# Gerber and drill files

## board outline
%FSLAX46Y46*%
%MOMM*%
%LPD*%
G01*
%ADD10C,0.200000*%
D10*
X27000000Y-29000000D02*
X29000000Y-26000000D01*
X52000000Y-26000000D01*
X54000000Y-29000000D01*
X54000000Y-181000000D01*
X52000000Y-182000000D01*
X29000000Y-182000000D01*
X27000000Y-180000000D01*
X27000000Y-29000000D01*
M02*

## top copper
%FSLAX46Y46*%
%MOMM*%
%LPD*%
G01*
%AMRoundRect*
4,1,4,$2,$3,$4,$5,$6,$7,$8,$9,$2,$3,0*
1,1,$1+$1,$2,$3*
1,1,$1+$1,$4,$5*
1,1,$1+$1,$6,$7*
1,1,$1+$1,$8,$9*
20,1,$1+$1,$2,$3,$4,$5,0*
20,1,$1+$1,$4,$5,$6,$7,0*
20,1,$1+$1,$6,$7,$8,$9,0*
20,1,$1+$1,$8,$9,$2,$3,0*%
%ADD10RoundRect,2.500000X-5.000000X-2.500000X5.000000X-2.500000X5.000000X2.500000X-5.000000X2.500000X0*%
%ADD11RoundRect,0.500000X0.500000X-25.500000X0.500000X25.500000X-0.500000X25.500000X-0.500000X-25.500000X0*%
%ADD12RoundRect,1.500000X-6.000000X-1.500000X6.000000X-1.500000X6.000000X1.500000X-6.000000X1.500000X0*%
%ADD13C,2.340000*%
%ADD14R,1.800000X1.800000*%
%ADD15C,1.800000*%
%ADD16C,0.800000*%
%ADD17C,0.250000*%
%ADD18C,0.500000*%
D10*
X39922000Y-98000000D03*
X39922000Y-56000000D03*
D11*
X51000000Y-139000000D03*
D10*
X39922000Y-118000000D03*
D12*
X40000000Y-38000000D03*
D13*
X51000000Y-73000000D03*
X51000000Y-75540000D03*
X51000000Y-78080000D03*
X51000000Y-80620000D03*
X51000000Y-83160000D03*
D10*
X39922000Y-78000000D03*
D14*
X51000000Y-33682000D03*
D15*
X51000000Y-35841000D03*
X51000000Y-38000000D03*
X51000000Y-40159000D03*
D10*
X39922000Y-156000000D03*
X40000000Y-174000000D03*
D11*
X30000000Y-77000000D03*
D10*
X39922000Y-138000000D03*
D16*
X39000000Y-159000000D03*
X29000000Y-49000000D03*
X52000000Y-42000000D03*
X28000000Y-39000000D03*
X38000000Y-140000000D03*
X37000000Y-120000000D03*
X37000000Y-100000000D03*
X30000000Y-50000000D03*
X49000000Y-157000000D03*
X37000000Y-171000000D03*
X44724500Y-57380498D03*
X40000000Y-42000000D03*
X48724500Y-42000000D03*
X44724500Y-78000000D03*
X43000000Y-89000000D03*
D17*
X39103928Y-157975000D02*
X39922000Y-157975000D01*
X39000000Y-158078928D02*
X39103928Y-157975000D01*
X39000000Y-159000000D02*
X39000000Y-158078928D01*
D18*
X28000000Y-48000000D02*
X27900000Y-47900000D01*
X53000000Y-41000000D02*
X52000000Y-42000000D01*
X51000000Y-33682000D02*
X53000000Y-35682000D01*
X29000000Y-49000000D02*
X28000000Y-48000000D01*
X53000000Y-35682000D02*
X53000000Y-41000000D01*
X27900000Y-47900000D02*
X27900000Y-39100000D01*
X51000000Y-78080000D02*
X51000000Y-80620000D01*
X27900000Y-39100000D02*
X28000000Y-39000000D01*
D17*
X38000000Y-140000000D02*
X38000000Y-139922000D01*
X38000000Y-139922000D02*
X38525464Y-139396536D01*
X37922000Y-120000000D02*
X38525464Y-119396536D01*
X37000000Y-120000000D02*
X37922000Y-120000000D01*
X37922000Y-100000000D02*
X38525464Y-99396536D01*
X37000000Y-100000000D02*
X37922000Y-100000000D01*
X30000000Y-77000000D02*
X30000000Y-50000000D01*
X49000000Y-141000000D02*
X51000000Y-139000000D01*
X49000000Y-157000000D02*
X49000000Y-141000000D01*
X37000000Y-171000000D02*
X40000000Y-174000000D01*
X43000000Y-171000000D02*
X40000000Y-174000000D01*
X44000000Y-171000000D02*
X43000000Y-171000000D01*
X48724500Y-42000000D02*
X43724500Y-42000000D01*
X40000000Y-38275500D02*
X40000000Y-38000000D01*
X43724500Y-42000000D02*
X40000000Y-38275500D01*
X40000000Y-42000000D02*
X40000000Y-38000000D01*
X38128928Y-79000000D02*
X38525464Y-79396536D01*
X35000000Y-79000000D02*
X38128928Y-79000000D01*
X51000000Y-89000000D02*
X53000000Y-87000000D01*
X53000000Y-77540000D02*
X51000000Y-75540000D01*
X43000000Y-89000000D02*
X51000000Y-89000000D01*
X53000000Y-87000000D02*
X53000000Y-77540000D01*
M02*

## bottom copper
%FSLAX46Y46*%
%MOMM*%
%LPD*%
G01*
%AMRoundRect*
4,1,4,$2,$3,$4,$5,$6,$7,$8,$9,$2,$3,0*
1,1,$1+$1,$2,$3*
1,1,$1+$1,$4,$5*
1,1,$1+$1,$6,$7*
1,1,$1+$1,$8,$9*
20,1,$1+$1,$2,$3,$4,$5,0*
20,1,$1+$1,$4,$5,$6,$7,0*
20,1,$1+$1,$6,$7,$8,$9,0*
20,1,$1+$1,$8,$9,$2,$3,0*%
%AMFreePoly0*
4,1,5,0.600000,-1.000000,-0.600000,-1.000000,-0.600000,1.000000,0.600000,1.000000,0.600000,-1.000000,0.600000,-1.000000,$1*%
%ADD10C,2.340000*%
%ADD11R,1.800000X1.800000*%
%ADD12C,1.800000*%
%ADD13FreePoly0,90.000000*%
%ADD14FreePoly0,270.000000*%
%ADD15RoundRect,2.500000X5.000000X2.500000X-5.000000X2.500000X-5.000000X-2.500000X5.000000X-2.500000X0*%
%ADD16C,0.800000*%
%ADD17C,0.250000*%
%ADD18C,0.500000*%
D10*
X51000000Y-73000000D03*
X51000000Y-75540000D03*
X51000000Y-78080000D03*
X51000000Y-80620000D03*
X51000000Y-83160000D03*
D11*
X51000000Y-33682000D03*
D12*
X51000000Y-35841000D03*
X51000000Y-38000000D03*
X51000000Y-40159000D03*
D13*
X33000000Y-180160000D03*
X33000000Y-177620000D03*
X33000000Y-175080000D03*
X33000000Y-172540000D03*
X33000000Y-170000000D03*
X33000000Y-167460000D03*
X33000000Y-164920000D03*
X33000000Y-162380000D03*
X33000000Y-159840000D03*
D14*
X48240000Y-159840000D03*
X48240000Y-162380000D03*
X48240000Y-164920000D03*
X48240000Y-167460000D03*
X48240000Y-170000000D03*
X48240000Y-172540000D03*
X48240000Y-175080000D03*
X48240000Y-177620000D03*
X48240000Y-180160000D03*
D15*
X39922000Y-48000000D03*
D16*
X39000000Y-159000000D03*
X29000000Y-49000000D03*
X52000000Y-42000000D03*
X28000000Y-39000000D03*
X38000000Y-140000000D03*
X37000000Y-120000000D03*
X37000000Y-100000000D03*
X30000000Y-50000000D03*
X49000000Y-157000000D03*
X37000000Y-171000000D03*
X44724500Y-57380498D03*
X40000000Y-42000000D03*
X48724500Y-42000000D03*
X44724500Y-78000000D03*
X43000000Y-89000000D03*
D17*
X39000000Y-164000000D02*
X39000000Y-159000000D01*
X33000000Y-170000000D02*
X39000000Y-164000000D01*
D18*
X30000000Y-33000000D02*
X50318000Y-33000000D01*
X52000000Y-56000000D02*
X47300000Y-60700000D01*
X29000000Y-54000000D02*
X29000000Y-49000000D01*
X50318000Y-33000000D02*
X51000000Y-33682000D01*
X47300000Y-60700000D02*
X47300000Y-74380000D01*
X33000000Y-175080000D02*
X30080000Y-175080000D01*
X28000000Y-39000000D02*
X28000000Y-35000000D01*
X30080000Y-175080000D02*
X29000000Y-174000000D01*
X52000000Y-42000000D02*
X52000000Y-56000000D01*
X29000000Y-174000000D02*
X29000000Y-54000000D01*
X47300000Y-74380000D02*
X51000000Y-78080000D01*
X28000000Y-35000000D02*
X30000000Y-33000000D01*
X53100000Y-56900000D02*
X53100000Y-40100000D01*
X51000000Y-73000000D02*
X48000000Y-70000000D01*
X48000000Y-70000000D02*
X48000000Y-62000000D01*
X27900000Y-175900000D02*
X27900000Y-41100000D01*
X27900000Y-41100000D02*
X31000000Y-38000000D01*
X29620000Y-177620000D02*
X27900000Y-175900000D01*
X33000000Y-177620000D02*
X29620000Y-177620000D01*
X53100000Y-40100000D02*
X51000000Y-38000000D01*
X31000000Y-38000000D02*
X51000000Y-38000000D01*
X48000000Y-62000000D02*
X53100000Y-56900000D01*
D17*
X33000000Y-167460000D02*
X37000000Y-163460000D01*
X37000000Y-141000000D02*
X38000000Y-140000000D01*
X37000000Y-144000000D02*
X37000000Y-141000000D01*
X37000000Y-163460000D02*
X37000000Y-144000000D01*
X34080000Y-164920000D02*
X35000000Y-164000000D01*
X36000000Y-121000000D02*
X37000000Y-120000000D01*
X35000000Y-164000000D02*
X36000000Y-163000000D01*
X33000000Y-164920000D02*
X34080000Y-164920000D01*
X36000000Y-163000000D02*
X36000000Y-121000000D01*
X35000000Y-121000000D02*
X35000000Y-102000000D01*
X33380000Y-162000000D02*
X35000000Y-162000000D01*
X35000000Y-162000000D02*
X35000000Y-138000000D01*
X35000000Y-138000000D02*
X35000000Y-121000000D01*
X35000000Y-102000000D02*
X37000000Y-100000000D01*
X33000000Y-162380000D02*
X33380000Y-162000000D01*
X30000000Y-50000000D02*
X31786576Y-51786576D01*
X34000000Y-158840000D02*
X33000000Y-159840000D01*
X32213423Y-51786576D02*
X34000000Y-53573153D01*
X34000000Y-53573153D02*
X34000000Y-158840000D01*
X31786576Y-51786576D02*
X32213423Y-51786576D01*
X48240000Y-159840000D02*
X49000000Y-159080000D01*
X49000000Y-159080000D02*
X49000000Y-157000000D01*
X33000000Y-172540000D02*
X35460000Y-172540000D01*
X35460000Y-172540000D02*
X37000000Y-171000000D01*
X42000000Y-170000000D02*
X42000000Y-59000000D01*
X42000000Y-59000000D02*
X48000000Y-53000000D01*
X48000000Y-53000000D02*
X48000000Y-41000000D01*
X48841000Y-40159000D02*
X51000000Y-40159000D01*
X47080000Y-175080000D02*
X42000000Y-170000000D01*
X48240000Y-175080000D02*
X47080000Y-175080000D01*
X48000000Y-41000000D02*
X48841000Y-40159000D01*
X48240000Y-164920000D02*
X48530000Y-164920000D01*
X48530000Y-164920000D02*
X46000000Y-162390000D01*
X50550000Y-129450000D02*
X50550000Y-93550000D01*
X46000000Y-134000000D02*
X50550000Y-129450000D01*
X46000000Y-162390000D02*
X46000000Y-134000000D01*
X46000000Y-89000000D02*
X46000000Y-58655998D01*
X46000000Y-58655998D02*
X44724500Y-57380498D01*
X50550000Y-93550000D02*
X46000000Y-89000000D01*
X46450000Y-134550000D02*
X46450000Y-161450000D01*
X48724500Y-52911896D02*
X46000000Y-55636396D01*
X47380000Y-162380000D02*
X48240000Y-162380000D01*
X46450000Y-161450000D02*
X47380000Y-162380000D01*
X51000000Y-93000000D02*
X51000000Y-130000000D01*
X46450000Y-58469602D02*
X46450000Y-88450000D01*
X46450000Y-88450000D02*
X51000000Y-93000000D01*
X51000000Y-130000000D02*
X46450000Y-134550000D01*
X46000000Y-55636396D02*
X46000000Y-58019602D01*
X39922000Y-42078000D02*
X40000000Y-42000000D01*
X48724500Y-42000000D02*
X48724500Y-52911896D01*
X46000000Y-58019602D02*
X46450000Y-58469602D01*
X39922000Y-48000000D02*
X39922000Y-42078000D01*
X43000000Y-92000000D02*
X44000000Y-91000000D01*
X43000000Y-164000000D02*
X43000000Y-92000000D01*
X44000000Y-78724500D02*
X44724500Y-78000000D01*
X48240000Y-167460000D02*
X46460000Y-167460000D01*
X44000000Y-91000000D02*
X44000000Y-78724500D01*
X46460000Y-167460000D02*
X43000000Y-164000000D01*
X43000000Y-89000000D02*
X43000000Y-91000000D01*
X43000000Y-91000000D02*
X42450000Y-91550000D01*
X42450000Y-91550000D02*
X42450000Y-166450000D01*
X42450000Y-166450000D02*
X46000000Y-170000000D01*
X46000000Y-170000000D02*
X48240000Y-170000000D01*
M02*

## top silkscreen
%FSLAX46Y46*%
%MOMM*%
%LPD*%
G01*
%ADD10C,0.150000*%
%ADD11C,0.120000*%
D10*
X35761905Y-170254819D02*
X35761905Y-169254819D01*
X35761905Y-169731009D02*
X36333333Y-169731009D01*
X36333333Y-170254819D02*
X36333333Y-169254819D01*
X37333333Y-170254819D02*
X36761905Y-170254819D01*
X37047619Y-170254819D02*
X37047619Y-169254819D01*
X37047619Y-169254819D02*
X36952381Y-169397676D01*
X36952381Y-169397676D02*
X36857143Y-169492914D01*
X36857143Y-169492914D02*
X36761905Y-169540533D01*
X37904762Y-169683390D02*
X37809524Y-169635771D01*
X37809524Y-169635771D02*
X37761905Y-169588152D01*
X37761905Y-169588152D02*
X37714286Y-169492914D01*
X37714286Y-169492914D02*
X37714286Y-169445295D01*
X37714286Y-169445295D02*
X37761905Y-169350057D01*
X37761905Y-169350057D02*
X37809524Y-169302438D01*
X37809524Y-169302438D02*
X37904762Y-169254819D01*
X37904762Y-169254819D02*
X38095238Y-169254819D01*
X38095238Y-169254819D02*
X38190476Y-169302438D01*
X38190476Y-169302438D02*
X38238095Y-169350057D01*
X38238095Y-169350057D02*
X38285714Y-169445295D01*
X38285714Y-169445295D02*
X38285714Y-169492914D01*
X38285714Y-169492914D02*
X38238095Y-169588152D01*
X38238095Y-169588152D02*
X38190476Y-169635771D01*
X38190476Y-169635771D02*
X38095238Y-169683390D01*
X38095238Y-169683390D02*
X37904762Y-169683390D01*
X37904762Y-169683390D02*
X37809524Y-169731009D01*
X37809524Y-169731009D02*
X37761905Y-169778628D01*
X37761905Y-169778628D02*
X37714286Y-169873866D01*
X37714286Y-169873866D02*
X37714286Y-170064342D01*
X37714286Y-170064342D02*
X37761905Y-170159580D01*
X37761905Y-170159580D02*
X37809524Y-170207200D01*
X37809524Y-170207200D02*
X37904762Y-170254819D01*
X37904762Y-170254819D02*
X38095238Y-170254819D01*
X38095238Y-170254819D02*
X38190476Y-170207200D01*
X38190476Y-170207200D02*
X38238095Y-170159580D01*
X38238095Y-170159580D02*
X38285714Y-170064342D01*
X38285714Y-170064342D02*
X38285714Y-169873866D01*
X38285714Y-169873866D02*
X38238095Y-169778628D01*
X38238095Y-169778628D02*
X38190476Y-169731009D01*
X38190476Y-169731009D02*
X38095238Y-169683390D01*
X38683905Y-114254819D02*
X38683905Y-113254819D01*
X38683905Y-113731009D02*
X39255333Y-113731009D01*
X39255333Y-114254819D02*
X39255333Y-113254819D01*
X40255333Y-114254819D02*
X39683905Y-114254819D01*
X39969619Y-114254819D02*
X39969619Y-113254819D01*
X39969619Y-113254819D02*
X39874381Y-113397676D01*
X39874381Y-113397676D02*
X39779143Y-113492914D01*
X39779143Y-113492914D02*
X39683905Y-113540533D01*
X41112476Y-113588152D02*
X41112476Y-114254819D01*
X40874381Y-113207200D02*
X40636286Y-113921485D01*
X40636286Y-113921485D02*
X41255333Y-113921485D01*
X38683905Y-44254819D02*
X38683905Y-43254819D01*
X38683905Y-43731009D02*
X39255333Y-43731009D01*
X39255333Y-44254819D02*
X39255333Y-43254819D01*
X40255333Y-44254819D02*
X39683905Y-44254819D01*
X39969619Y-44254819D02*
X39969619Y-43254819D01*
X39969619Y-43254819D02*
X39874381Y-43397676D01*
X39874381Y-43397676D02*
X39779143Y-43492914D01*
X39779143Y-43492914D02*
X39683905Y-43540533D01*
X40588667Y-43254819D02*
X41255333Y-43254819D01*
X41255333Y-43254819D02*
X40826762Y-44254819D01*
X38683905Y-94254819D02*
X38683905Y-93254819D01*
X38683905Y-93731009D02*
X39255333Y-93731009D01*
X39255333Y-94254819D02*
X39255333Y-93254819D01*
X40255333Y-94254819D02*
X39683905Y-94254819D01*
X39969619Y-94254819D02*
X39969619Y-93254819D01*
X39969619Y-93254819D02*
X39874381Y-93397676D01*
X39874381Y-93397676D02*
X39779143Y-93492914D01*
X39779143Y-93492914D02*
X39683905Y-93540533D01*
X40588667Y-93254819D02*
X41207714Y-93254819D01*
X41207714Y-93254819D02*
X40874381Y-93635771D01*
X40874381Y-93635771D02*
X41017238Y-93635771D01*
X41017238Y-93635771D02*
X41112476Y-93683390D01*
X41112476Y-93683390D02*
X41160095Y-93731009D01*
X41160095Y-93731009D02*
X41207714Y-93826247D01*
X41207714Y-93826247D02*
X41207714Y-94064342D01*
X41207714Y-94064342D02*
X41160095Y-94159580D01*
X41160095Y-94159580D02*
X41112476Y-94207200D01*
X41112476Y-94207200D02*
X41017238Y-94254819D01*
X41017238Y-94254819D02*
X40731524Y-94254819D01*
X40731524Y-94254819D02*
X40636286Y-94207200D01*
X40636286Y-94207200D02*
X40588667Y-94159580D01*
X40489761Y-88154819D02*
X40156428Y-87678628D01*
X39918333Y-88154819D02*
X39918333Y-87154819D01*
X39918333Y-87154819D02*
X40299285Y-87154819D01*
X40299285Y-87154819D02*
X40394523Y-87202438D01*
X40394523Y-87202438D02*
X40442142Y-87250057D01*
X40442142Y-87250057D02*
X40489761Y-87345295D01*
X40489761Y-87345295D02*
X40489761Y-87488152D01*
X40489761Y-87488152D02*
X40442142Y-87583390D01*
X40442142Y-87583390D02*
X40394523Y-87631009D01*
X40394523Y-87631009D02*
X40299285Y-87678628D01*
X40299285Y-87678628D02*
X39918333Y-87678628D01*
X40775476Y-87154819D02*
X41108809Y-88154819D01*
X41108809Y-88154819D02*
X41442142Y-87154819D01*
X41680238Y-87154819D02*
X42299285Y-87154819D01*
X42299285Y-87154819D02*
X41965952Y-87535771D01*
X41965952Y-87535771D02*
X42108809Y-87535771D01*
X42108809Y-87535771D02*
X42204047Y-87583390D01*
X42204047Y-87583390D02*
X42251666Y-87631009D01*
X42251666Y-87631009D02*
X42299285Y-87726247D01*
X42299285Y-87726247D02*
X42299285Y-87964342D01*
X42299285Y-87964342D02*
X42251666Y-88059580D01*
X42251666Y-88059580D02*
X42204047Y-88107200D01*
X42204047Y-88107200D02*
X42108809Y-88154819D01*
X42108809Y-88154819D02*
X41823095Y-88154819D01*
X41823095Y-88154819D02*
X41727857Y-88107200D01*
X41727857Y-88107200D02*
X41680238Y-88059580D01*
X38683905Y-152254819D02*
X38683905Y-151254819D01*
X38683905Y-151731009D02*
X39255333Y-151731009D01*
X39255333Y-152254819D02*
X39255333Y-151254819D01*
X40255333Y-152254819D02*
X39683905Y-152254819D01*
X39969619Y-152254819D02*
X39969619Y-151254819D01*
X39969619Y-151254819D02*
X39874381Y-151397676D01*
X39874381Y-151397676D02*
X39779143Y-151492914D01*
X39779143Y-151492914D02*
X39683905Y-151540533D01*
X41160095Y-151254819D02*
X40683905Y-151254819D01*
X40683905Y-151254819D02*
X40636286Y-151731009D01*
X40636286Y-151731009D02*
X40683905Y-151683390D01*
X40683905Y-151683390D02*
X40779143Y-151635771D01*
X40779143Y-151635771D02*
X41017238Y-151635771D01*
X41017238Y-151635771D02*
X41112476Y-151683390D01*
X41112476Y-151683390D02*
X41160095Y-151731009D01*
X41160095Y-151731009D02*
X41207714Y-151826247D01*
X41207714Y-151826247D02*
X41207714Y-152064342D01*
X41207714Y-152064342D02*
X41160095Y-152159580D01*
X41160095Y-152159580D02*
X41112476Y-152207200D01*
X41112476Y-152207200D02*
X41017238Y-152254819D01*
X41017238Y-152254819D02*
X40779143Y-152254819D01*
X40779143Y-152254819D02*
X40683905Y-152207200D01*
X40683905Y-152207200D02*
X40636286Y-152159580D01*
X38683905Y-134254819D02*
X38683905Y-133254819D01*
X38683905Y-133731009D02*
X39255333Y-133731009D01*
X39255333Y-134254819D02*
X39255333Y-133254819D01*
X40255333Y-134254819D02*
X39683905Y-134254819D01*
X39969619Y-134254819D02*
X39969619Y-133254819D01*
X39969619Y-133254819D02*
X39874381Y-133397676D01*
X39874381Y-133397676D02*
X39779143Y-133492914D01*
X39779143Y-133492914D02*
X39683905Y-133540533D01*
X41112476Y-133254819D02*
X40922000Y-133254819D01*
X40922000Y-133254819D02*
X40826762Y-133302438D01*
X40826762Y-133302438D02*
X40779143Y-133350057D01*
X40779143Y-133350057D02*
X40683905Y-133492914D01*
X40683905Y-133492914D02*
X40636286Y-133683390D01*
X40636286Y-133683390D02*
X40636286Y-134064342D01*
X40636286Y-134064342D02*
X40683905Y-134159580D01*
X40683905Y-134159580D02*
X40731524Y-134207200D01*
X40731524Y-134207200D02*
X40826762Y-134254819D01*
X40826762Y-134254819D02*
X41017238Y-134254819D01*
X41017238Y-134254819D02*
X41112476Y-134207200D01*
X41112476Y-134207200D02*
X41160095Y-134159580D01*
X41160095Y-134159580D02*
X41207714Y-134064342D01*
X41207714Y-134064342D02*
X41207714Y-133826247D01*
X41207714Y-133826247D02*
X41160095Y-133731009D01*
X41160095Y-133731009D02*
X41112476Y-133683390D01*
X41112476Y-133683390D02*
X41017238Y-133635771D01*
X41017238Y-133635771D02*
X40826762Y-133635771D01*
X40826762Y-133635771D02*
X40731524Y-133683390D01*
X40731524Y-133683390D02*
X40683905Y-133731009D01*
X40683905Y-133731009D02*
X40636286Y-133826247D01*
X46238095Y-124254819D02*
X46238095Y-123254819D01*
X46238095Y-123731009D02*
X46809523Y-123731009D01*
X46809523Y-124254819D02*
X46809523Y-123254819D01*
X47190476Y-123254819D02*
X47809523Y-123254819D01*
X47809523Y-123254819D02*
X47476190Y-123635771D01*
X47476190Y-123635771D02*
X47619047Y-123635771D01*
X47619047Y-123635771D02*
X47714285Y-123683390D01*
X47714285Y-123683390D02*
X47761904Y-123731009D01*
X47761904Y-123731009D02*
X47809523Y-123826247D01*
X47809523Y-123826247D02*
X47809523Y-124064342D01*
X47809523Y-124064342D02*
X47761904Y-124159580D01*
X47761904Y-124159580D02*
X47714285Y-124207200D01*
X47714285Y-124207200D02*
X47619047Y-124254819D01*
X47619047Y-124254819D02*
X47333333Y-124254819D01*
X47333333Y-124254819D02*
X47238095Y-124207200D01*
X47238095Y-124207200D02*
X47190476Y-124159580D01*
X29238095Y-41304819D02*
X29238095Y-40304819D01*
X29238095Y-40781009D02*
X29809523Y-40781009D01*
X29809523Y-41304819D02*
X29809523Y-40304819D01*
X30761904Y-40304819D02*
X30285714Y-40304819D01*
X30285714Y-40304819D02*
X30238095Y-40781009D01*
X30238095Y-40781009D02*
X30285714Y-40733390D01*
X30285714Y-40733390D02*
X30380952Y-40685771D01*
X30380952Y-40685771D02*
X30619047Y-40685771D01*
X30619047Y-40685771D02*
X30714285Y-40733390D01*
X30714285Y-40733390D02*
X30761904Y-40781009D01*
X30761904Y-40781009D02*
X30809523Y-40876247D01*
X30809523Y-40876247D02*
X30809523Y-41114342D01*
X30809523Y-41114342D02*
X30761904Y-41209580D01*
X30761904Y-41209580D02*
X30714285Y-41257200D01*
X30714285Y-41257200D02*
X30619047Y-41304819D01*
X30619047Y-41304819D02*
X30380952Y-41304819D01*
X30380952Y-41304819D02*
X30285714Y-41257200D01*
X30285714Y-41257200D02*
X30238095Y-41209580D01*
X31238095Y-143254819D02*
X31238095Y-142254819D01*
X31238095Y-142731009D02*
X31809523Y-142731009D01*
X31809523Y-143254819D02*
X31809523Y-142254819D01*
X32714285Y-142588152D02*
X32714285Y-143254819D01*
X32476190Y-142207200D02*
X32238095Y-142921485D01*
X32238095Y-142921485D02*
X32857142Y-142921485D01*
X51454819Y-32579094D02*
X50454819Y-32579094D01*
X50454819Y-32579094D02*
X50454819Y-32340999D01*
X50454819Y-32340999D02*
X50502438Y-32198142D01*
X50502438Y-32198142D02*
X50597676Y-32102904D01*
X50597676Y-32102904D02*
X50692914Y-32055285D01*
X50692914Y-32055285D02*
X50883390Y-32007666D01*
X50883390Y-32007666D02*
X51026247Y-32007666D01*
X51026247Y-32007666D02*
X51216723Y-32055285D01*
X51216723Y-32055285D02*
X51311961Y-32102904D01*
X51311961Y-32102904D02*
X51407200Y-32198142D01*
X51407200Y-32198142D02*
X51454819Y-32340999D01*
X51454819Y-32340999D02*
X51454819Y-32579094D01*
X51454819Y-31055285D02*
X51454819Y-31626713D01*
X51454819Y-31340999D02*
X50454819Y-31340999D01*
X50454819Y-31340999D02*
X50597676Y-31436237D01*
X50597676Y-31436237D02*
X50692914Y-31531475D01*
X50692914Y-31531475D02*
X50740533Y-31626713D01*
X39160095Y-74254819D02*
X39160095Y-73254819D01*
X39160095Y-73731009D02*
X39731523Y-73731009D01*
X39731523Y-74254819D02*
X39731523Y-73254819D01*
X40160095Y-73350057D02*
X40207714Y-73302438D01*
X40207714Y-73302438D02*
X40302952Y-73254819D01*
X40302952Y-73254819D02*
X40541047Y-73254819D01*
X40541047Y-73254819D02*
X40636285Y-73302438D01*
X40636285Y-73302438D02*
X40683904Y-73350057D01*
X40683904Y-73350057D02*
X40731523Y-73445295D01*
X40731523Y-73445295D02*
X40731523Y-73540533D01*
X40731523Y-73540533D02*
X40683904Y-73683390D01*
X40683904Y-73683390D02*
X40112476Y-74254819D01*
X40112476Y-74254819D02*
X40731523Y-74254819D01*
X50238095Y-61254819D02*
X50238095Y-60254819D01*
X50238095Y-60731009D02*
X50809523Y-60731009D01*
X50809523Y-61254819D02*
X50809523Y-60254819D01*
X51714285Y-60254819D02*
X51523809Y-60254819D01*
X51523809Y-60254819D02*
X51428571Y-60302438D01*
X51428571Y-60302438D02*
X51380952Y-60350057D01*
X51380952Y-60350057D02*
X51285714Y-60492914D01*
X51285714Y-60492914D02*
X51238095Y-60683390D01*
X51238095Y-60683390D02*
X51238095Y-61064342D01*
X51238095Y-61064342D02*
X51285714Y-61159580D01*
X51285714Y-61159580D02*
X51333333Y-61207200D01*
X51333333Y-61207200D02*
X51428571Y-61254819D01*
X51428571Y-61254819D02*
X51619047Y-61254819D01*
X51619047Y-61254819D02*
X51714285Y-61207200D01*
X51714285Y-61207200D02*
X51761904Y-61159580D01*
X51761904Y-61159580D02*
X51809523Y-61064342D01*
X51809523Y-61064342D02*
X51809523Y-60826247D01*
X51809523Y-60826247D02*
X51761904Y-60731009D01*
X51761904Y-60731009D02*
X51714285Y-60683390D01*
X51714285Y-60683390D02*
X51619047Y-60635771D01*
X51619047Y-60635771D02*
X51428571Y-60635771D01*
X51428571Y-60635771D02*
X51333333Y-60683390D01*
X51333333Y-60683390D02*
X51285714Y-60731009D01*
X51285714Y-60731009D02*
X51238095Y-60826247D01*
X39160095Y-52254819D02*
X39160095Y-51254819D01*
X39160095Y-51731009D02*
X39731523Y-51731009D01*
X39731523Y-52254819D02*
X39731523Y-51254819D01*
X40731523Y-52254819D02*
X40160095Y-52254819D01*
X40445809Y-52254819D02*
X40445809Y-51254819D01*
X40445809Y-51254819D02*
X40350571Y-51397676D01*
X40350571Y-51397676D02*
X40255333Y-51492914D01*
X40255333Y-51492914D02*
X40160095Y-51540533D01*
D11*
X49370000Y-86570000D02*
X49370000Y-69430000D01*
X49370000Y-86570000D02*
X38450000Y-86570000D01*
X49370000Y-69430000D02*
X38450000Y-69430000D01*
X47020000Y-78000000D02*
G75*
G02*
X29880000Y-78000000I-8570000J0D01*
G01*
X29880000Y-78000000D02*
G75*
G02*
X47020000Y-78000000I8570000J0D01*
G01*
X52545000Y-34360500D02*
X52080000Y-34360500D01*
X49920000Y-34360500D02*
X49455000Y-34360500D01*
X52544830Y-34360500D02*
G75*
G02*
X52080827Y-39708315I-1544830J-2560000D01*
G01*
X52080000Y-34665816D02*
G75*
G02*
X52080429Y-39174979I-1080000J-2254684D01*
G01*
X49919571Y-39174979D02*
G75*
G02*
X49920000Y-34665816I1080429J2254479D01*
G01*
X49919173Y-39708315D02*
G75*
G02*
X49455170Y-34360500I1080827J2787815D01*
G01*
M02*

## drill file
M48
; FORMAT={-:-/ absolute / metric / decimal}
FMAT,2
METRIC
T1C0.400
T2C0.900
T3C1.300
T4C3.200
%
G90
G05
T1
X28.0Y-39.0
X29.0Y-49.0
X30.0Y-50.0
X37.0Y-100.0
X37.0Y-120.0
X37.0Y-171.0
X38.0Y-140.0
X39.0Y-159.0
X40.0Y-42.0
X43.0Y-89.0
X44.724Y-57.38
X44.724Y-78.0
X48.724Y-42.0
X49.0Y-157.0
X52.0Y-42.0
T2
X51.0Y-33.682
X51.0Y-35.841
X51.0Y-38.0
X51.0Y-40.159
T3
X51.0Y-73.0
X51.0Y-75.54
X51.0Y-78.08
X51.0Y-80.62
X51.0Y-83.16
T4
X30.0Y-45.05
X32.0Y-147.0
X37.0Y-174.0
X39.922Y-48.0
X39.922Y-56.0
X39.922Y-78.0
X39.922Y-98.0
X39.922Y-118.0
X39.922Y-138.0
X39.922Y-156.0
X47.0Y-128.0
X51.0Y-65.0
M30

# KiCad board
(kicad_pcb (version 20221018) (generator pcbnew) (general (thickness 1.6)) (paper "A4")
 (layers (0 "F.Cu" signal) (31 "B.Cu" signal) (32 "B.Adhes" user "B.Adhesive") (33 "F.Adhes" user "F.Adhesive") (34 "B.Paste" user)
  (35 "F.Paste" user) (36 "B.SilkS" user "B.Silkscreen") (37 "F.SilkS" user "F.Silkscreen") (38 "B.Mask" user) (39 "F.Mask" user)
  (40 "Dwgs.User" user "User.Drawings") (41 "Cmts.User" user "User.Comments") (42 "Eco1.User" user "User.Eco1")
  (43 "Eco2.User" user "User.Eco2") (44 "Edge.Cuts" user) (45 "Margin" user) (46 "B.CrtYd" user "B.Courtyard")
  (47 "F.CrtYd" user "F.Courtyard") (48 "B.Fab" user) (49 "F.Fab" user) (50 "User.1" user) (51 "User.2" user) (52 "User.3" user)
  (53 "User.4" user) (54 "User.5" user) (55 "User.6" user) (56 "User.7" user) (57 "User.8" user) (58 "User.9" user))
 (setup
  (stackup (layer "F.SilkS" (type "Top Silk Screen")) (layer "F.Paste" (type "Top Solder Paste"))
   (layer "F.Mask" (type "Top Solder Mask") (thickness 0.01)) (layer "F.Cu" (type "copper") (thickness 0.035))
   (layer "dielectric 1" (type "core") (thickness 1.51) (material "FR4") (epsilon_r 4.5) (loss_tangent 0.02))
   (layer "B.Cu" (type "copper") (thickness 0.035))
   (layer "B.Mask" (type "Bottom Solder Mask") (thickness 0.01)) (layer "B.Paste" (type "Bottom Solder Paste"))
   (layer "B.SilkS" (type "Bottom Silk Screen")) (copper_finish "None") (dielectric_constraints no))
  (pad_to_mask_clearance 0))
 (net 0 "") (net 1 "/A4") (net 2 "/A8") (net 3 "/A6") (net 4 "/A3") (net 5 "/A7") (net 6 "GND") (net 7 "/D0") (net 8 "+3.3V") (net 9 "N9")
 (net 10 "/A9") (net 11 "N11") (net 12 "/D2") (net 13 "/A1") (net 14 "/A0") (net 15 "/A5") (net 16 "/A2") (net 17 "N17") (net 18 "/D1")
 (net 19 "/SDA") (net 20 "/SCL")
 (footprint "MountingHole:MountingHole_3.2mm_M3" (layer "F.Cu") (at 37 174)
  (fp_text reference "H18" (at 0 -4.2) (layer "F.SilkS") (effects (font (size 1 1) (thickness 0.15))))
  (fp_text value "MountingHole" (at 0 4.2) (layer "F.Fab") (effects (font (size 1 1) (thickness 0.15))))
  (pad "" np_thru_hole circle (at 0 0) (size 3.2 3.2) (drill 3.2) (layers "*.Cu" "*.Mask")))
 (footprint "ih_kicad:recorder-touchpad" (layer "F.Cu") (at 39.922 98)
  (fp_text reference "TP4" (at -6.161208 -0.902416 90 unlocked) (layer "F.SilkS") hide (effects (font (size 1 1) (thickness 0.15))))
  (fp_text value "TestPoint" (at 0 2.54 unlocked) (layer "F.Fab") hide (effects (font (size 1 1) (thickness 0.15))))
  (pad "1" smd roundrect (at 0 0) (size 15 10) (layers "F.Cu" "F.Mask") (roundrect_rratio 0.25) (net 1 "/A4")))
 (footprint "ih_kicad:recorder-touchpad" (layer "F.Cu") (at 39.922 56)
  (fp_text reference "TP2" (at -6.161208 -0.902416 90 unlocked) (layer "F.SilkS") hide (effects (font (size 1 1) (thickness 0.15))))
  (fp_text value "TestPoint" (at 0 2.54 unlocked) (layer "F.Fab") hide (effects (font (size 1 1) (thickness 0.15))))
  (pad "1" smd roundrect (at 0 0) (size 15 10) (layers "F.Cu" "F.Mask") (roundrect_rratio 0.25) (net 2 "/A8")))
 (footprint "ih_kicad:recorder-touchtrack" (layer "F.Cu") (at 51 139 90)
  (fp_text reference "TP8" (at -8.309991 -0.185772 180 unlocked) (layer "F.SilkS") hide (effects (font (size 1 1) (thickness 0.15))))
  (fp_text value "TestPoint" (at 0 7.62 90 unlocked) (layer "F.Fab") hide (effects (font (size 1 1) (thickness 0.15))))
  (pad "1" smd roundrect (at 0 0 90) (size 52 2) (layers "F.Cu" "F.Mask") (roundrect_rratio 0.25) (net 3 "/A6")))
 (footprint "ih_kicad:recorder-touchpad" (layer "F.Cu") (at 39.922 118)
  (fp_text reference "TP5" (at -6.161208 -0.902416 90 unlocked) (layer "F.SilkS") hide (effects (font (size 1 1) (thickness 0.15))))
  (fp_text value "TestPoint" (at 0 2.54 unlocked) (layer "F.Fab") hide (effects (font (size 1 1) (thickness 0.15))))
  (pad "1" smd roundrect (at 0 0) (size 15 10) (layers "F.Cu" "F.Mask") (roundrect_rratio 0.25) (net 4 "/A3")))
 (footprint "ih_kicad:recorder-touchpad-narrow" (layer "F.Cu") (at 40 38)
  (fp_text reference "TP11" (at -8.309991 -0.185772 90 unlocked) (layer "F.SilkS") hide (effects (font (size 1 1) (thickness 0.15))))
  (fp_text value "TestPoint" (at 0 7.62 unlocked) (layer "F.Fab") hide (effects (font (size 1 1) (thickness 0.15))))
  (pad "1" smd roundrect (at 0 0) (size 15 6) (layers "F.Cu" "F.Mask") (roundrect_rratio 0.25) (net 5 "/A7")))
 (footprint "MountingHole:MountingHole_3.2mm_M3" (layer "F.Cu") (at 39.922 118)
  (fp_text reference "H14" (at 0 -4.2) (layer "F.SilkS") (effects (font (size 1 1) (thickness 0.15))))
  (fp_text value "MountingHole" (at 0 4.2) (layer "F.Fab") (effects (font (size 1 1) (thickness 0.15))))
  (pad "" np_thru_hole circle (at 0 0) (size 3.2 3.2) (drill 3.2) (layers "*.Cu" "*.Mask")))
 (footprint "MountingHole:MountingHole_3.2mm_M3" (layer "F.Cu") (at 39.922 48)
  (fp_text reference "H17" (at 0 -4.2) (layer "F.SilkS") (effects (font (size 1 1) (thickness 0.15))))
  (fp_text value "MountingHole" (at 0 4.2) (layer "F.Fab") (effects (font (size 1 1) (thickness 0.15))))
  (pad "" np_thru_hole circle (at 0 0) (size 3.2 3.2) (drill 3.2) (layers "*.Cu" "*.Mask")))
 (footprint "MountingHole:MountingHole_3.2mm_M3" (layer "F.Cu") (at 39.922 98)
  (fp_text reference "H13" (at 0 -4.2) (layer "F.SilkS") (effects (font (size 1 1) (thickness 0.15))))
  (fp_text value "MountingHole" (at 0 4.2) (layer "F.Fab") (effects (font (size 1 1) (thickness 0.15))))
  (pad "" np_thru_hole circle (at 0 0) (size 3.2 3.2) (drill 3.2) (layers "*.Cu" "*.Mask")))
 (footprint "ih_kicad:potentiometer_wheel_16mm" (layer "F.Cu") (at 51 73 180)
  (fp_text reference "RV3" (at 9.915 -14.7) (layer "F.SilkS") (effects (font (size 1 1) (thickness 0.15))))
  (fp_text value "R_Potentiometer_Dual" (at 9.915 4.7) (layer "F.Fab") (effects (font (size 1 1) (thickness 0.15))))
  (fp_line (start 1.63 -13.57) (end 1.63 3.57) (stroke (width 0.12) (type solid)) (layer "F.SilkS"))
  (fp_line (start 1.63 -13.57) (end 12.55 -13.57) (stroke (width 0.12) (type solid)) (layer "F.SilkS"))
  (fp_line (start 1.63 3.57) (end 12.55 3.57) (stroke (width 0.12) (type solid)) (layer "F.SilkS"))
  (fp_circle (center 12.55 -5) (end 21.12 -5) (stroke (width 0.12) (type solid)) (fill none) (layer "F.SilkS"))
  (pad "1" thru_hole circle (at 0 0 180) (size 2.34 2.34) (drill 1.3) (layers "*.Cu" "*.Mask") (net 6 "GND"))
  (pad "2" thru_hole circle (at 0 -2.54 180) (size 2.34 2.34) (drill 1.3) (layers "*.Cu" "*.Mask") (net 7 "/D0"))
  (pad "3" thru_hole circle (at 0 -5.08 180) (size 2.34 2.34) (drill 1.3) (layers "*.Cu" "*.Mask") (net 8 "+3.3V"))
  (pad "4" thru_hole circle (at 0 -7.62 180) (size 2.34 2.34) (drill 1.3) (layers "*.Cu" "*.Mask") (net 8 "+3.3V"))
  (pad "5" thru_hole circle (at 0 -10.16 180) (size 2.34 2.34) (drill 1.3) (layers "*.Cu" "*.Mask") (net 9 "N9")))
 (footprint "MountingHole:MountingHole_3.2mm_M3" (layer "F.Cu") (at 39.922 156)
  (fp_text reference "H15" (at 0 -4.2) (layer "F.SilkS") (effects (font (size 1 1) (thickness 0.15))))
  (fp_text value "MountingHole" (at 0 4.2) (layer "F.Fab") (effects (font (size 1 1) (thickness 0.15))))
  (pad "" np_thru_hole circle (at 0 0) (size 3.2 3.2) (drill 3.2) (layers "*.Cu" "*.Mask")))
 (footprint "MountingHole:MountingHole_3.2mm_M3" (layer "F.Cu") (at 39.922 138)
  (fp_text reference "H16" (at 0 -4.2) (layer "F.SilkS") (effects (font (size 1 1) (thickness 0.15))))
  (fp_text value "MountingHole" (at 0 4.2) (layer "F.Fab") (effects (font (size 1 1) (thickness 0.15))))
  (pad "" np_thru_hole circle (at 0 0) (size 3.2 3.2) (drill 3.2) (layers "*.Cu" "*.Mask")))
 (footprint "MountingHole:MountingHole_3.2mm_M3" (layer "F.Cu") (at 47 128)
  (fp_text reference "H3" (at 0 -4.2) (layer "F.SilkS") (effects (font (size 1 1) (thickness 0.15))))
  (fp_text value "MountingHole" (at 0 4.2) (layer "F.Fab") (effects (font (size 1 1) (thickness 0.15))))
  (pad "" np_thru_hole circle (at 0 0) (size 3.2 3.2) (drill 3.2) (layers "*.Cu" "*.Mask")))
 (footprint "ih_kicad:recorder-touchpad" (layer "F.Cu") (at 39.922 78)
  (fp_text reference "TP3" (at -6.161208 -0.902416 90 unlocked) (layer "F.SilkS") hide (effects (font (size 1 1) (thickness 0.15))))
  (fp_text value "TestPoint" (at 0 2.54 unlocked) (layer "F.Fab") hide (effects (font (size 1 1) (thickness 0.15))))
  (pad "1" smd roundrect (at 0 0) (size 15 10) (layers "F.Cu" "F.Mask") (roundrect_rratio 0.25) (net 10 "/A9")))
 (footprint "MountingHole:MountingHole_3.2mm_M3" (layer "F.Cu") (at 30 45.05)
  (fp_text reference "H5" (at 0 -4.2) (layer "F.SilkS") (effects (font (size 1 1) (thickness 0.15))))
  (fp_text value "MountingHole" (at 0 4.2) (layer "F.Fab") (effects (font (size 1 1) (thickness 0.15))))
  (pad "" np_thru_hole circle (at 0 0) (size 3.2 3.2) (drill 3.2) (layers "*.Cu" "*.Mask")))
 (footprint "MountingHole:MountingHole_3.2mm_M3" (layer "F.Cu") (at 32 147)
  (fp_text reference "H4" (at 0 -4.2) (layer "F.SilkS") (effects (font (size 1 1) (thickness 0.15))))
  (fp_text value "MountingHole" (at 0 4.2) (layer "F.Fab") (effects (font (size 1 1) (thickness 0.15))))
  (pad "" np_thru_hole circle (at 0 0) (size 3.2 3.2) (drill 3.2) (layers "*.Cu" "*.Mask")))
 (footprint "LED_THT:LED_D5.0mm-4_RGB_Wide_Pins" (layer "F.Cu") (at 51 33.682 -90)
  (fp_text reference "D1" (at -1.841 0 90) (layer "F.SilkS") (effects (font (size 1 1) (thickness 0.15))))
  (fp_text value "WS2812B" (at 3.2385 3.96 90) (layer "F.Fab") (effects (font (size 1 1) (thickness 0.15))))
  (fp_line (start 0.6785 -1.545) (end 0.6785 -1.08) (stroke (width 0.12) (type solid)) (layer "F.SilkS"))
  (fp_line (start 0.6785 1.08) (end 0.6785 1.545) (stroke (width 0.12) (type solid)) (layer "F.SilkS"))
  (fp_arc (start 0.6785 -1.54483) (mid 3.496956 -2.978809) (end 6.026315 -1.080827) (stroke (width 0.12) (type solid)) (layer "F.SilkS"))
  (fp_arc (start 0.983816 -1.08) (mid 3.238262 -2.5) (end 5.492979 -1.080429) (stroke (width 0.12) (type solid)) (layer "F.SilkS"))
  (fp_arc (start 5.492979 1.080429) (mid 3.238262 2.5) (end 0.983816 1.08) (stroke (width 0.12) (type solid)) (layer "F.SilkS"))
  (fp_arc (start 6.026315 1.080827) (mid 3.496956 2.978808) (end 0.6785 1.54483) (stroke (width 0.12) (type solid)) (layer "F.SilkS"))
  (pad "1" thru_hole rect (at 0 0 270) (size 1.8 1.8) (drill 0.9) (layers "*.Cu" "*.Mask") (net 8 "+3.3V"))
  (pad "2" thru_hole circle (at 2.159 0 270) (size 1.8 1.8) (drill 0.9) (layers "*.Cu" "*.Mask") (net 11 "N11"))
  (pad "3" thru_hole circle (at 4.318 0 270) (size 1.8 1.8) (drill 0.9) (layers "*.Cu" "*.Mask") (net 6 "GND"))
  (pad "4" thru_hole circle (at 6.477 0 270) (size 1.8 1.8) (drill 0.9) (layers "*.Cu" "*.Mask") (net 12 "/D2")))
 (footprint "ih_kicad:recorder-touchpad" (layer "F.Cu") (at 39.922 156)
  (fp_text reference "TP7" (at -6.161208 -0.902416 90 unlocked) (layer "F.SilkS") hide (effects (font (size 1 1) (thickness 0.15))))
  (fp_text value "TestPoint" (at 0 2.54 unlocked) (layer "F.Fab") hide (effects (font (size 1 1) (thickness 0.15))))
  (pad "1" smd roundrect (at 0 0) (size 15 10) (layers "F.Cu" "F.Mask") (roundrect_rratio 0.25) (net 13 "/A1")))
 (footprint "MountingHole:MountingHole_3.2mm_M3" (layer "F.Cu") (at 39.922 78)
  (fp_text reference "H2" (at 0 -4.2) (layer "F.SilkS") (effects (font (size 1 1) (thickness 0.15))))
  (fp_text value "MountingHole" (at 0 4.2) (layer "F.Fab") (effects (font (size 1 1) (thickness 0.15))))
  (pad "" np_thru_hole circle (at 0 0) (size 3.2 3.2) (drill 3.2) (layers "*.Cu" "*.Mask")))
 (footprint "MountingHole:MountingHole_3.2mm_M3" (layer "F.Cu") (at 51 65)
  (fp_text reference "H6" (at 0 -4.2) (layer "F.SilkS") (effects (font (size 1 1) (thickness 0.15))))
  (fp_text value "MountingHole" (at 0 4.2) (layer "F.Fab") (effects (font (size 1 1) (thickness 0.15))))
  (pad "" np_thru_hole circle (at 0 0) (size 3.2 3.2) (drill 3.2) (layers "*.Cu" "*.Mask")))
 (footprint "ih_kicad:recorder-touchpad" (layer "F.Cu") (at 40 174)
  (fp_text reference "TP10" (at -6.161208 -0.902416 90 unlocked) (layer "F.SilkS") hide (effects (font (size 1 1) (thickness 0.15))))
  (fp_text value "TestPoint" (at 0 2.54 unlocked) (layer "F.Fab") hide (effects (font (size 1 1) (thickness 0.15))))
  (pad "1" smd roundrect (at 0 0) (size 15 10) (layers "F.Cu" "F.Mask") (roundrect_rratio 0.25) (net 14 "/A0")))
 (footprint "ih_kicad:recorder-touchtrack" (layer "F.Cu") (at 30 77 90)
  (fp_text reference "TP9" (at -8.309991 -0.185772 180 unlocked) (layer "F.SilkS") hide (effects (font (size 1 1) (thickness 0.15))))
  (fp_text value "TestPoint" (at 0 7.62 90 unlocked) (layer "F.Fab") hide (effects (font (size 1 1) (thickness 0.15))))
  (pad "1" smd roundrect (at 0 0 90) (size 52 2) (layers "F.Cu" "F.Mask") (roundrect_rratio 0.25) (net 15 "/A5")))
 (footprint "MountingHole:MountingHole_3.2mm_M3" (layer "F.Cu") (at 39.922 56)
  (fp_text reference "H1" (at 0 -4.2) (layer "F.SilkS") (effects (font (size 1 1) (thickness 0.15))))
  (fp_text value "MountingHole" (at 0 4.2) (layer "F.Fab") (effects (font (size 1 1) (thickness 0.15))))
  (pad "" np_thru_hole circle (at 0 0) (size 3.2 3.2) (drill 3.2) (layers "*.Cu" "*.Mask")))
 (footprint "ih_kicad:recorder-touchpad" (layer "F.Cu") (at 39.922 138)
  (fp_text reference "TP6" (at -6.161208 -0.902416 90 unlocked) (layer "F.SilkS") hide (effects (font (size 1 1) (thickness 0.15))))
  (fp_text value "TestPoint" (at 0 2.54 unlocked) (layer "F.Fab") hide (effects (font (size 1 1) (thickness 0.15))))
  (pad "1" smd roundrect (at 0 0) (size 15 10) (layers "F.Cu" "F.Mask") (roundrect_rratio 0.25) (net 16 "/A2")))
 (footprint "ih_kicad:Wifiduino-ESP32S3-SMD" (layer "B.Cu") (at 40.62 170)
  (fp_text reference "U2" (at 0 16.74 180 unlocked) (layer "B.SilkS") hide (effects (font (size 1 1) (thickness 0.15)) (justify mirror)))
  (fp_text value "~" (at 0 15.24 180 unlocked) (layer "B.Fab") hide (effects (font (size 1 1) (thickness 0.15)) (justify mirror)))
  (pad "1" smd custom (at -7.62 10.16 90) (size 1.2 2) (layers "B.Cu" "B.Paste" "B.Mask") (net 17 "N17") (thermal_bridge_angle 45)
   (options (clearance outline) (anchor rect)) (primitives))
  (pad "2" smd custom (at -7.62 7.62 90) (size 1.2 2) (layers "B.Cu" "B.Paste" "B.Mask") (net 6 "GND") (thermal_bridge_angle 45)
   (options (clearance outline) (anchor rect)) (primitives))
  (pad "3" smd custom (at -7.62 5.08 90) (size 1.2 2) (layers "B.Cu" "B.Paste" "B.Mask") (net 8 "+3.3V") (thermal_bridge_angle 45)
   (options (clearance outline) (anchor rect)) (primitives))
  (pad "4" smd custom (at -7.62 2.54 90) (size 1.2 2) (layers "B.Cu" "B.Paste" "B.Mask") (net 14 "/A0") (thermal_bridge_angle 45)
   (options (clearance outline) (anchor rect)) (primitives))
  (pad "5" smd custom (at -7.62 0 90) (size 1.2 2) (layers "B.Cu" "B.Paste" "B.Mask") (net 13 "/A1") (thermal_bridge_angle 45)
   (options (clearance outline) (anchor rect)) (primitives))
  (pad "6" smd custom (at -7.62 -2.54 90) (size 1.2 2) (layers "B.Cu" "B.Paste" "B.Mask") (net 16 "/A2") (thermal_bridge_angle 45)
   (options (clearance outline) (anchor rect)) (primitives))
  (pad "7" smd custom (at -7.62 -5.08 90) (size 1.2 2) (layers "B.Cu" "B.Paste" "B.Mask") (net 4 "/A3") (thermal_bridge_angle 45)
   (options (clearance outline) (anchor rect)) (primitives))
  (pad "8" smd custom (at -7.62 -7.62 90) (size 1.2 2) (layers "B.Cu" "B.Paste" "B.Mask") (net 1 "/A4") (thermal_bridge_angle 45)
   (options (clearance outline) (anchor rect)) (primitives))
  (pad "9" smd custom (at -7.62 -10.16 90) (size 1.2 2) (layers "B.Cu" "B.Paste" "B.Mask") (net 15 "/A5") (thermal_bridge_angle 45)
   (options (clearance outline) (anchor rect)) (primitives))
  (pad "10" smd custom (at 7.62 -10.16 270) (size 1.2 2) (layers "B.Cu" "B.Paste" "B.Mask") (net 3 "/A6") (thermal_bridge_angle 45)
   (options (clearance outline) (anchor rect)) (primitives))
  (pad "11" smd custom (at 7.62 -7.62 270) (size 1.2 2) (layers "B.Cu" "B.Paste" "B.Mask") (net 5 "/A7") (thermal_bridge_angle 45)
   (options (clearance outline) (anchor rect)) (primitives))
  (pad "12" smd custom (at 7.62 -5.08 270) (size 1.2 2) (layers "B.Cu" "B.Paste" "B.Mask") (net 2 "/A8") (thermal_bridge_angle 45)
   (options (clearance outline) (anchor rect)) (primitives))
  (pad "13" smd custom (at 7.62 -2.54 270) (size 1.2 2) (layers "B.Cu" "B.Paste" "B.Mask") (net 10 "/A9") (thermal_bridge_angle 45)
   (options (clearance outline) (anchor rect)) (primitives))
  (pad "14" smd custom (at 7.62 0 270) (size 1.2 2) (layers "B.Cu" "B.Paste" "B.Mask") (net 7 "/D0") (thermal_bridge_angle 45)
   (options (clearance outline) (anchor rect)) (primitives))
  (pad "15" smd custom (at 7.62 2.54 270) (size 1.2 2) (layers "B.Cu" "B.Paste" "B.Mask") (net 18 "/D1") (thermal_bridge_angle 45)
   (options (clearance outline) (anchor rect)) (primitives))
  (pad "16" smd custom (at 7.62 5.08 270) (size 1.2 2) (layers "B.Cu" "B.Paste" "B.Mask") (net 12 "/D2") (thermal_bridge_angle 45)
   (options (clearance outline) (anchor rect)) (primitives))
  (pad "17" smd custom (at 7.62 7.62 270) (size 1.2 2) (layers "B.Cu" "B.Paste" "B.Mask") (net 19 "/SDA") (thermal_bridge_angle 45)
   (options (clearance outline) (anchor rect)) (primitives))
  (pad "18" smd custom (at 7.62 10.16 270) (size 1.2 2) (layers "B.Cu" "B.Paste" "B.Mask") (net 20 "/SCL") (thermal_bridge_angle 45)
   (options (clearance outline) (anchor rect)) (primitives)))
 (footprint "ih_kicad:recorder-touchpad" (layer "B.Cu") (at 39.922 48 180)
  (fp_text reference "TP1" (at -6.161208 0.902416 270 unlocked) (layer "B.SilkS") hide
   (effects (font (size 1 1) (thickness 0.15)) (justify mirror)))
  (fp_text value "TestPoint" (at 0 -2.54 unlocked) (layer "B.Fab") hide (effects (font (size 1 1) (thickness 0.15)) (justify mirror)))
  (pad "1" smd roundrect (at 0 0 180) (size 15 10) (layers "B.Cu" "B.Mask") (roundrect_rratio 0.25) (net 5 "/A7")))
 (gr_poly
  (pts (xy 27 29) (xy 29 26) (xy 52 26) (xy 54 29) (xy 54 181) (xy 52 182) (xy 29 182) (xy 27 180)) (stroke (width 0.2) (type solid))
  (fill none) (layer "Edge.Cuts"))
 (segment (start 39.103928 157.975) (end 39.922 157.975) (width 0.25) (layer "F.Cu") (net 13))
 (segment (start 39 158.078928) (end 39.103928 157.975) (width 0.25) (layer "F.Cu") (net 13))
 (segment (start 39 159) (end 39 158.078928) (width 0.25) (layer "F.Cu") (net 13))
 (via (at 39 159) (size 0.8) (drill 0.4) (layers "F.Cu" "B.Cu") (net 13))
 (segment (start 39 164) (end 39 159) (width 0.25) (layer "B.Cu") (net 13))
 (segment (start 33 170) (end 39 164) (width 0.25) (layer "B.Cu") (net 13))
 (segment (start 28 48) (end 27.9 47.9) (width 0.5) (layer "F.Cu") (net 8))
 (segment (start 53 41) (end 52 42) (width 0.5) (layer "F.Cu") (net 8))
 (segment (start 51 33.682) (end 53 35.682) (width 0.5) (layer "F.Cu") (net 8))
 (segment (start 29 49) (end 28 48) (width 0.5) (layer "F.Cu") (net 8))
 (segment (start 53 35.682) (end 53 41) (width 0.5) (layer "F.Cu") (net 8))
 (segment (start 27.9 47.9) (end 27.9 39.1) (width 0.5) (layer "F.Cu") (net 8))
 (segment (start 51 78.08) (end 51 80.62) (width 0.5) (layer "F.Cu") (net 8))
 (segment (start 27.9 39.1) (end 28 39) (width 0.5) (layer "F.Cu") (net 8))
 (via (at 29 49) (size 0.8) (drill 0.4) (layers "F.Cu" "B.Cu") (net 8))
 (via (at 52 42) (size 0.8) (drill 0.4) (layers "F.Cu" "B.Cu") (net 8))
 (via (at 28 39) (size 0.8) (drill 0.4) (layers "F.Cu" "B.Cu") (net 8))
 (segment (start 30 33) (end 50.318 33) (width 0.5) (layer "B.Cu") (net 8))
 (segment (start 52 56) (end 47.3 60.7) (width 0.5) (layer "B.Cu") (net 8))
 (segment (start 29 54) (end 29 49) (width 0.5) (layer "B.Cu") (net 8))
 (segment (start 50.318 33) (end 51 33.682) (width 0.5) (layer "B.Cu") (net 8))
 (segment (start 47.3 60.7) (end 47.3 74.38) (width 0.5) (layer "B.Cu") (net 8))
 (segment (start 33 175.08) (end 30.08 175.08) (width 0.5) (layer "B.Cu") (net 8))
 (segment (start 28 39) (end 28 35) (width 0.5) (layer "B.Cu") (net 8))
 (segment (start 30.08 175.08) (end 29 174) (width 0.5) (layer "B.Cu") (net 8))
 (segment (start 52 42) (end 52 56) (width 0.5) (layer "B.Cu") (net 8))
 (segment (start 29 174) (end 29 54) (width 0.5) (layer "B.Cu") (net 8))
 (segment (start 47.3 74.38) (end 51 78.08) (width 0.5) (layer "B.Cu") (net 8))
 (segment (start 28 35) (end 30 33) (width 0.5) (layer "B.Cu") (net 8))
 (segment (start 53.1 56.9) (end 53.1 40.1) (width 0.5) (layer "B.Cu") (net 6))
 (segment (start 51 73) (end 48 70) (width 0.5) (layer "B.Cu") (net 6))
 (segment (start 48 70) (end 48 62) (width 0.5) (layer "B.Cu") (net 6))
 (segment (start 27.9 175.9) (end 27.9 41.1) (width 0.5) (layer "B.Cu") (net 6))
 (segment (start 27.9 41.1) (end 31 38) (width 0.5) (layer "B.Cu") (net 6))
 (segment (start 29.62 177.62) (end 27.9 175.9) (width 0.5) (layer "B.Cu") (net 6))
 (segment (start 33 177.62) (end 29.62 177.62) (width 0.5) (layer "B.Cu") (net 6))
 (segment (start 53.1 40.1) (end 51 38) (width 0.5) (layer "B.Cu") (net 6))
 (segment (start 31 38) (end 51 38) (width 0.5) (layer "B.Cu") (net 6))
 (segment (start 48 62) (end 53.1 56.9) (width 0.5) (layer "B.Cu") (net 6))
 (segment (start 38 140) (end 38 139.922) (width 0.25) (layer "F.Cu") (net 16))
 (segment (start 38 139.922) (end 38.525464 139.396536) (width 0.25) (layer "F.Cu") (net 16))
 (via (at 38 140) (size 0.8) (drill 0.4) (layers "F.Cu" "B.Cu") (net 16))
 (segment (start 33 167.46) (end 37 163.46) (width 0.25) (layer "B.Cu") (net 16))
 (segment (start 37 141) (end 38 140) (width 0.25) (layer "B.Cu") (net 16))
 (segment (start 37 144) (end 37 141) (width 0.25) (layer "B.Cu") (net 16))
 (segment (start 37 163.46) (end 37 144) (width 0.25) (layer "B.Cu") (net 16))
 (segment (start 37.922 120) (end 38.525464 119.396536) (width 0.25) (layer "F.Cu") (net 4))
 (segment (start 37 120) (end 37.922 120) (width 0.25) (layer "F.Cu") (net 4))
 (via (at 37 120) (size 0.8) (drill 0.4) (layers "F.Cu" "B.Cu") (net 4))
 (segment (start 34.08 164.92) (end 35 164) (width 0.25) (layer "B.Cu") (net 4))
 (segment (start 36 121) (end 37 120) (width 0.25) (layer "B.Cu") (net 4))
 (segment (start 35 164) (end 36 163) (width 0.25) (layer "B.Cu") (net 4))
 (segment (start 33 164.92) (end 34.08 164.92) (width 0.25) (layer "B.Cu") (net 4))
 (segment (start 36 163) (end 36 121) (width 0.25) (layer "B.Cu") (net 4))
 (segment (start 37.922 100) (end 38.525464 99.396536) (width 0.25) (layer "F.Cu") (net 1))
 (segment (start 37 100) (end 37.922 100) (width 0.25) (layer "F.Cu") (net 1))
 (via (at 37 100) (size 0.8) (drill 0.4) (layers "F.Cu" "B.Cu") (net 1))
 (segment (start 35 121) (end 35 102) (width 0.25) (layer "B.Cu") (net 1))
 (segment (start 33.38 162) (end 35 162) (width 0.25) (layer "B.Cu") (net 1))
 (segment (start 35 162) (end 35 138) (width 0.25) (layer "B.Cu") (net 1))
 (segment (start 35 138) (end 35 121) (width 0.25) (layer "B.Cu") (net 1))
 (segment (start 35 102) (end 37 100) (width 0.25) (layer "B.Cu") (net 1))
 (segment (start 33 162.38) (end 33.38 162) (width 0.25) (layer "B.Cu") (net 1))
 (segment (start 30 77) (end 30 50) (width 0.25) (layer "F.Cu") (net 15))
 (via (at 30 50) (size 0.8) (drill 0.4) (layers "F.Cu" "B.Cu") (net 15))
 (segment (start 30 50) (end 31.786576 51.786576) (width 0.25) (layer "B.Cu") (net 15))
 (segment (start 34 158.84) (end 33 159.84) (width 0.25) (layer "B.Cu") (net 15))
 (segment (start 32.213423 51.786576) (end 34 53.573153) (width 0.25) (layer "B.Cu") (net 15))
 (segment (start 34 53.573153) (end 34 158.84) (width 0.25) (layer "B.Cu") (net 15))
 (segment (start 31.786576 51.786576) (end 32.213423 51.786576) (width 0.25) (layer "B.Cu") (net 15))
 (segment (start 49 141) (end 51 139) (width 0.25) (layer "F.Cu") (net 3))
 (segment (start 49 157) (end 49 141) (width 0.25) (layer "F.Cu") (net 3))
 (via (at 49 157) (size 0.8) (drill 0.4) (layers "F.Cu" "B.Cu") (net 3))
 (segment (start 48.24 159.84) (end 49 159.08) (width 0.25) (layer "B.Cu") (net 3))
 (segment (start 49 159.08) (end 49 157) (width 0.25) (layer "B.Cu") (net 3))
 (segment (start 37 171) (end 40 174) (width 0.25) (layer "F.Cu") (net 14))
 (segment (start 43 171) (end 40 174) (width 0.25) (layer "F.Cu") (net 14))
 (segment (start 44 171) (end 43 171) (width 0.25) (layer "F.Cu") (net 14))
 (via (at 37 171) (size 0.8) (drill 0.4) (layers "F.Cu" "B.Cu") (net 14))
 (segment (start 33 172.54) (end 35.46 172.54) (width 0.25) (layer "B.Cu") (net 14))
 (segment (start 35.46 172.54) (end 37 171) (width 0.25) (layer "B.Cu") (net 14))
 (segment (start 42 170) (end 42 59) (width 0.25) (layer "B.Cu") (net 12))
 (segment (start 42 59) (end 48 53) (width 0.25) (layer "B.Cu") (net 12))
 (segment (start 48 53) (end 48 41) (width 0.25) (layer "B.Cu") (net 12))
 (segment (start 48.841 40.159) (end 51 40.159) (width 0.25) (layer "B.Cu") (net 12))
 (segment (start 47.08 175.08) (end 42 170) (width 0.25) (layer "B.Cu") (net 12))
 (segment (start 48.24 175.08) (end 47.08 175.08) (width 0.25) (layer "B.Cu") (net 12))
 (segment (start 48 41) (end 48.841 40.159) (width 0.25) (layer "B.Cu") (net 12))
 (via (at 44.7245 57.380498) (size 0.8) (drill 0.4) (layers "F.Cu" "B.Cu") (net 2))
 (segment (start 48.24 164.92) (end 48.53 164.92) (width 0.25) (layer "B.Cu") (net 2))
 (segment (start 48.53 164.92) (end 46 162.39) (width 0.25) (layer "B.Cu") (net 2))
 (segment (start 50.55 129.45) (end 50.55 93.55) (width 0.25) (layer "B.Cu") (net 2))
 (segment (start 46 134) (end 50.55 129.45) (width 0.25) (layer "B.Cu") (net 2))
 (segment (start 46 162.39) (end 46 134) (width 0.25) (layer "B.Cu") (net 2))
 (segment (start 46 89) (end 46 58.655998) (width 0.25) (layer "B.Cu") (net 2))
 (segment (start 46 58.655998) (end 44.7245 57.380498) (width 0.25) (layer "B.Cu") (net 2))
 (segment (start 50.55 93.55) (end 46 89) (width 0.25) (layer "B.Cu") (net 2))
 (segment (start 48.7245 42) (end 43.7245 42) (width 0.25) (layer "F.Cu") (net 5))
 (segment (start 40 38.2755) (end 40 38) (width 0.25) (layer "F.Cu") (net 5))
 (segment (start 43.7245 42) (end 40 38.2755) (width 0.25) (layer "F.Cu") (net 5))
 (segment (start 40 42) (end 40 38) (width 0.25) (layer "F.Cu") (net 5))
 (via (at 40 42) (size 0.8) (drill 0.4) (layers "F.Cu" "B.Cu") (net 5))
 (via (at 48.7245 42) (size 0.8) (drill 0.4) (layers "F.Cu" "B.Cu") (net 5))
 (segment (start 46.45 134.55) (end 46.45 161.45) (width 0.25) (layer "B.Cu") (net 5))
 (segment (start 48.7245 52.911896) (end 46 55.636396) (width 0.25) (layer "B.Cu") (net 5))
 (segment (start 47.38 162.38) (end 48.24 162.38) (width 0.25) (layer "B.Cu") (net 5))
 (segment (start 46.45 161.45) (end 47.38 162.38) (width 0.25) (layer "B.Cu") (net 5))
 (segment (start 51 93) (end 51 130) (width 0.25) (layer "B.Cu") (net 5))
 (segment (start 46.45 58.469602) (end 46.45 88.45) (width 0.25) (layer "B.Cu") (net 5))
 (segment (start 46.45 88.45) (end 51 93) (width 0.25) (layer "B.Cu") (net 5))
 (segment (start 51 130) (end 46.45 134.55) (width 0.25) (layer "B.Cu") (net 5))
 (segment (start 46 55.636396) (end 46 58.019602) (width 0.25) (layer "B.Cu") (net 5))
 (segment (start 39.922 42.078) (end 40 42) (width 0.25) (layer "B.Cu") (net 5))
 (segment (start 48.7245 42) (end 48.7245 52.911896) (width 0.25) (layer "B.Cu") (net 5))
 (segment (start 46 58.019602) (end 46.45 58.469602) (width 0.25) (layer "B.Cu") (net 5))
 (segment (start 39.922 48) (end 39.922 42.078) (width 0.25) (layer "B.Cu") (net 5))
 (segment (start 38.128928 79) (end 38.525464 79.396536) (width 0.25) (layer "F.Cu") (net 10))
 (segment (start 35 79) (end 38.128928 79) (width 0.25) (layer "F.Cu") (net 10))
 (via (at 44.7245 78) (size 0.8) (drill 0.4) (layers "F.Cu" "B.Cu") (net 10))
 (segment (start 43 92) (end 44 91) (width 0.25) (layer "B.Cu") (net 10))
 (segment (start 43 164) (end 43 92) (width 0.25) (layer "B.Cu") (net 10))
 (segment (start 44 78.7245) (end 44.7245 78) (width 0.25) (layer "B.Cu") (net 10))
 (segment (start 48.24 167.46) (end 46.46 167.46) (width 0.25) (layer "B.Cu") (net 10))
 (segment (start 44 91) (end 44 78.7245) (width 0.25) (layer "B.Cu") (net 10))
 (segment (start 46.46 167.46) (end 43 164) (width 0.25) (layer "B.Cu") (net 10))
 (segment (start 51 89) (end 53 87) (width 0.25) (layer "F.Cu") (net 7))
 (segment (start 53 77.54) (end 51 75.54) (width 0.25) (layer "F.Cu") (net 7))
 (segment (start 43 89) (end 51 89) (width 0.25) (layer "F.Cu") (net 7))
 (segment (start 53 87) (end 53 77.54) (width 0.25) (layer "F.Cu") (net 7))
 (via (at 43 89) (size 0.8) (drill 0.4) (layers "F.Cu" "B.Cu") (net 7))
 (segment (start 43 89) (end 43 91) (width 0.25) (layer "B.Cu") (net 7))
 (segment (start 43 91) (end 42.45 91.55) (width 0.25) (layer "B.Cu") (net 7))
 (segment (start 42.45 91.55) (end 42.45 166.45) (width 0.25) (layer "B.Cu") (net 7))
 (segment (start 42.45 166.45) (end 46 170) (width 0.25) (layer "B.Cu") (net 7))
 (segment (start 46 170) (end 48.24 170) (width 0.25) (layer "B.Cu") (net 7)))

